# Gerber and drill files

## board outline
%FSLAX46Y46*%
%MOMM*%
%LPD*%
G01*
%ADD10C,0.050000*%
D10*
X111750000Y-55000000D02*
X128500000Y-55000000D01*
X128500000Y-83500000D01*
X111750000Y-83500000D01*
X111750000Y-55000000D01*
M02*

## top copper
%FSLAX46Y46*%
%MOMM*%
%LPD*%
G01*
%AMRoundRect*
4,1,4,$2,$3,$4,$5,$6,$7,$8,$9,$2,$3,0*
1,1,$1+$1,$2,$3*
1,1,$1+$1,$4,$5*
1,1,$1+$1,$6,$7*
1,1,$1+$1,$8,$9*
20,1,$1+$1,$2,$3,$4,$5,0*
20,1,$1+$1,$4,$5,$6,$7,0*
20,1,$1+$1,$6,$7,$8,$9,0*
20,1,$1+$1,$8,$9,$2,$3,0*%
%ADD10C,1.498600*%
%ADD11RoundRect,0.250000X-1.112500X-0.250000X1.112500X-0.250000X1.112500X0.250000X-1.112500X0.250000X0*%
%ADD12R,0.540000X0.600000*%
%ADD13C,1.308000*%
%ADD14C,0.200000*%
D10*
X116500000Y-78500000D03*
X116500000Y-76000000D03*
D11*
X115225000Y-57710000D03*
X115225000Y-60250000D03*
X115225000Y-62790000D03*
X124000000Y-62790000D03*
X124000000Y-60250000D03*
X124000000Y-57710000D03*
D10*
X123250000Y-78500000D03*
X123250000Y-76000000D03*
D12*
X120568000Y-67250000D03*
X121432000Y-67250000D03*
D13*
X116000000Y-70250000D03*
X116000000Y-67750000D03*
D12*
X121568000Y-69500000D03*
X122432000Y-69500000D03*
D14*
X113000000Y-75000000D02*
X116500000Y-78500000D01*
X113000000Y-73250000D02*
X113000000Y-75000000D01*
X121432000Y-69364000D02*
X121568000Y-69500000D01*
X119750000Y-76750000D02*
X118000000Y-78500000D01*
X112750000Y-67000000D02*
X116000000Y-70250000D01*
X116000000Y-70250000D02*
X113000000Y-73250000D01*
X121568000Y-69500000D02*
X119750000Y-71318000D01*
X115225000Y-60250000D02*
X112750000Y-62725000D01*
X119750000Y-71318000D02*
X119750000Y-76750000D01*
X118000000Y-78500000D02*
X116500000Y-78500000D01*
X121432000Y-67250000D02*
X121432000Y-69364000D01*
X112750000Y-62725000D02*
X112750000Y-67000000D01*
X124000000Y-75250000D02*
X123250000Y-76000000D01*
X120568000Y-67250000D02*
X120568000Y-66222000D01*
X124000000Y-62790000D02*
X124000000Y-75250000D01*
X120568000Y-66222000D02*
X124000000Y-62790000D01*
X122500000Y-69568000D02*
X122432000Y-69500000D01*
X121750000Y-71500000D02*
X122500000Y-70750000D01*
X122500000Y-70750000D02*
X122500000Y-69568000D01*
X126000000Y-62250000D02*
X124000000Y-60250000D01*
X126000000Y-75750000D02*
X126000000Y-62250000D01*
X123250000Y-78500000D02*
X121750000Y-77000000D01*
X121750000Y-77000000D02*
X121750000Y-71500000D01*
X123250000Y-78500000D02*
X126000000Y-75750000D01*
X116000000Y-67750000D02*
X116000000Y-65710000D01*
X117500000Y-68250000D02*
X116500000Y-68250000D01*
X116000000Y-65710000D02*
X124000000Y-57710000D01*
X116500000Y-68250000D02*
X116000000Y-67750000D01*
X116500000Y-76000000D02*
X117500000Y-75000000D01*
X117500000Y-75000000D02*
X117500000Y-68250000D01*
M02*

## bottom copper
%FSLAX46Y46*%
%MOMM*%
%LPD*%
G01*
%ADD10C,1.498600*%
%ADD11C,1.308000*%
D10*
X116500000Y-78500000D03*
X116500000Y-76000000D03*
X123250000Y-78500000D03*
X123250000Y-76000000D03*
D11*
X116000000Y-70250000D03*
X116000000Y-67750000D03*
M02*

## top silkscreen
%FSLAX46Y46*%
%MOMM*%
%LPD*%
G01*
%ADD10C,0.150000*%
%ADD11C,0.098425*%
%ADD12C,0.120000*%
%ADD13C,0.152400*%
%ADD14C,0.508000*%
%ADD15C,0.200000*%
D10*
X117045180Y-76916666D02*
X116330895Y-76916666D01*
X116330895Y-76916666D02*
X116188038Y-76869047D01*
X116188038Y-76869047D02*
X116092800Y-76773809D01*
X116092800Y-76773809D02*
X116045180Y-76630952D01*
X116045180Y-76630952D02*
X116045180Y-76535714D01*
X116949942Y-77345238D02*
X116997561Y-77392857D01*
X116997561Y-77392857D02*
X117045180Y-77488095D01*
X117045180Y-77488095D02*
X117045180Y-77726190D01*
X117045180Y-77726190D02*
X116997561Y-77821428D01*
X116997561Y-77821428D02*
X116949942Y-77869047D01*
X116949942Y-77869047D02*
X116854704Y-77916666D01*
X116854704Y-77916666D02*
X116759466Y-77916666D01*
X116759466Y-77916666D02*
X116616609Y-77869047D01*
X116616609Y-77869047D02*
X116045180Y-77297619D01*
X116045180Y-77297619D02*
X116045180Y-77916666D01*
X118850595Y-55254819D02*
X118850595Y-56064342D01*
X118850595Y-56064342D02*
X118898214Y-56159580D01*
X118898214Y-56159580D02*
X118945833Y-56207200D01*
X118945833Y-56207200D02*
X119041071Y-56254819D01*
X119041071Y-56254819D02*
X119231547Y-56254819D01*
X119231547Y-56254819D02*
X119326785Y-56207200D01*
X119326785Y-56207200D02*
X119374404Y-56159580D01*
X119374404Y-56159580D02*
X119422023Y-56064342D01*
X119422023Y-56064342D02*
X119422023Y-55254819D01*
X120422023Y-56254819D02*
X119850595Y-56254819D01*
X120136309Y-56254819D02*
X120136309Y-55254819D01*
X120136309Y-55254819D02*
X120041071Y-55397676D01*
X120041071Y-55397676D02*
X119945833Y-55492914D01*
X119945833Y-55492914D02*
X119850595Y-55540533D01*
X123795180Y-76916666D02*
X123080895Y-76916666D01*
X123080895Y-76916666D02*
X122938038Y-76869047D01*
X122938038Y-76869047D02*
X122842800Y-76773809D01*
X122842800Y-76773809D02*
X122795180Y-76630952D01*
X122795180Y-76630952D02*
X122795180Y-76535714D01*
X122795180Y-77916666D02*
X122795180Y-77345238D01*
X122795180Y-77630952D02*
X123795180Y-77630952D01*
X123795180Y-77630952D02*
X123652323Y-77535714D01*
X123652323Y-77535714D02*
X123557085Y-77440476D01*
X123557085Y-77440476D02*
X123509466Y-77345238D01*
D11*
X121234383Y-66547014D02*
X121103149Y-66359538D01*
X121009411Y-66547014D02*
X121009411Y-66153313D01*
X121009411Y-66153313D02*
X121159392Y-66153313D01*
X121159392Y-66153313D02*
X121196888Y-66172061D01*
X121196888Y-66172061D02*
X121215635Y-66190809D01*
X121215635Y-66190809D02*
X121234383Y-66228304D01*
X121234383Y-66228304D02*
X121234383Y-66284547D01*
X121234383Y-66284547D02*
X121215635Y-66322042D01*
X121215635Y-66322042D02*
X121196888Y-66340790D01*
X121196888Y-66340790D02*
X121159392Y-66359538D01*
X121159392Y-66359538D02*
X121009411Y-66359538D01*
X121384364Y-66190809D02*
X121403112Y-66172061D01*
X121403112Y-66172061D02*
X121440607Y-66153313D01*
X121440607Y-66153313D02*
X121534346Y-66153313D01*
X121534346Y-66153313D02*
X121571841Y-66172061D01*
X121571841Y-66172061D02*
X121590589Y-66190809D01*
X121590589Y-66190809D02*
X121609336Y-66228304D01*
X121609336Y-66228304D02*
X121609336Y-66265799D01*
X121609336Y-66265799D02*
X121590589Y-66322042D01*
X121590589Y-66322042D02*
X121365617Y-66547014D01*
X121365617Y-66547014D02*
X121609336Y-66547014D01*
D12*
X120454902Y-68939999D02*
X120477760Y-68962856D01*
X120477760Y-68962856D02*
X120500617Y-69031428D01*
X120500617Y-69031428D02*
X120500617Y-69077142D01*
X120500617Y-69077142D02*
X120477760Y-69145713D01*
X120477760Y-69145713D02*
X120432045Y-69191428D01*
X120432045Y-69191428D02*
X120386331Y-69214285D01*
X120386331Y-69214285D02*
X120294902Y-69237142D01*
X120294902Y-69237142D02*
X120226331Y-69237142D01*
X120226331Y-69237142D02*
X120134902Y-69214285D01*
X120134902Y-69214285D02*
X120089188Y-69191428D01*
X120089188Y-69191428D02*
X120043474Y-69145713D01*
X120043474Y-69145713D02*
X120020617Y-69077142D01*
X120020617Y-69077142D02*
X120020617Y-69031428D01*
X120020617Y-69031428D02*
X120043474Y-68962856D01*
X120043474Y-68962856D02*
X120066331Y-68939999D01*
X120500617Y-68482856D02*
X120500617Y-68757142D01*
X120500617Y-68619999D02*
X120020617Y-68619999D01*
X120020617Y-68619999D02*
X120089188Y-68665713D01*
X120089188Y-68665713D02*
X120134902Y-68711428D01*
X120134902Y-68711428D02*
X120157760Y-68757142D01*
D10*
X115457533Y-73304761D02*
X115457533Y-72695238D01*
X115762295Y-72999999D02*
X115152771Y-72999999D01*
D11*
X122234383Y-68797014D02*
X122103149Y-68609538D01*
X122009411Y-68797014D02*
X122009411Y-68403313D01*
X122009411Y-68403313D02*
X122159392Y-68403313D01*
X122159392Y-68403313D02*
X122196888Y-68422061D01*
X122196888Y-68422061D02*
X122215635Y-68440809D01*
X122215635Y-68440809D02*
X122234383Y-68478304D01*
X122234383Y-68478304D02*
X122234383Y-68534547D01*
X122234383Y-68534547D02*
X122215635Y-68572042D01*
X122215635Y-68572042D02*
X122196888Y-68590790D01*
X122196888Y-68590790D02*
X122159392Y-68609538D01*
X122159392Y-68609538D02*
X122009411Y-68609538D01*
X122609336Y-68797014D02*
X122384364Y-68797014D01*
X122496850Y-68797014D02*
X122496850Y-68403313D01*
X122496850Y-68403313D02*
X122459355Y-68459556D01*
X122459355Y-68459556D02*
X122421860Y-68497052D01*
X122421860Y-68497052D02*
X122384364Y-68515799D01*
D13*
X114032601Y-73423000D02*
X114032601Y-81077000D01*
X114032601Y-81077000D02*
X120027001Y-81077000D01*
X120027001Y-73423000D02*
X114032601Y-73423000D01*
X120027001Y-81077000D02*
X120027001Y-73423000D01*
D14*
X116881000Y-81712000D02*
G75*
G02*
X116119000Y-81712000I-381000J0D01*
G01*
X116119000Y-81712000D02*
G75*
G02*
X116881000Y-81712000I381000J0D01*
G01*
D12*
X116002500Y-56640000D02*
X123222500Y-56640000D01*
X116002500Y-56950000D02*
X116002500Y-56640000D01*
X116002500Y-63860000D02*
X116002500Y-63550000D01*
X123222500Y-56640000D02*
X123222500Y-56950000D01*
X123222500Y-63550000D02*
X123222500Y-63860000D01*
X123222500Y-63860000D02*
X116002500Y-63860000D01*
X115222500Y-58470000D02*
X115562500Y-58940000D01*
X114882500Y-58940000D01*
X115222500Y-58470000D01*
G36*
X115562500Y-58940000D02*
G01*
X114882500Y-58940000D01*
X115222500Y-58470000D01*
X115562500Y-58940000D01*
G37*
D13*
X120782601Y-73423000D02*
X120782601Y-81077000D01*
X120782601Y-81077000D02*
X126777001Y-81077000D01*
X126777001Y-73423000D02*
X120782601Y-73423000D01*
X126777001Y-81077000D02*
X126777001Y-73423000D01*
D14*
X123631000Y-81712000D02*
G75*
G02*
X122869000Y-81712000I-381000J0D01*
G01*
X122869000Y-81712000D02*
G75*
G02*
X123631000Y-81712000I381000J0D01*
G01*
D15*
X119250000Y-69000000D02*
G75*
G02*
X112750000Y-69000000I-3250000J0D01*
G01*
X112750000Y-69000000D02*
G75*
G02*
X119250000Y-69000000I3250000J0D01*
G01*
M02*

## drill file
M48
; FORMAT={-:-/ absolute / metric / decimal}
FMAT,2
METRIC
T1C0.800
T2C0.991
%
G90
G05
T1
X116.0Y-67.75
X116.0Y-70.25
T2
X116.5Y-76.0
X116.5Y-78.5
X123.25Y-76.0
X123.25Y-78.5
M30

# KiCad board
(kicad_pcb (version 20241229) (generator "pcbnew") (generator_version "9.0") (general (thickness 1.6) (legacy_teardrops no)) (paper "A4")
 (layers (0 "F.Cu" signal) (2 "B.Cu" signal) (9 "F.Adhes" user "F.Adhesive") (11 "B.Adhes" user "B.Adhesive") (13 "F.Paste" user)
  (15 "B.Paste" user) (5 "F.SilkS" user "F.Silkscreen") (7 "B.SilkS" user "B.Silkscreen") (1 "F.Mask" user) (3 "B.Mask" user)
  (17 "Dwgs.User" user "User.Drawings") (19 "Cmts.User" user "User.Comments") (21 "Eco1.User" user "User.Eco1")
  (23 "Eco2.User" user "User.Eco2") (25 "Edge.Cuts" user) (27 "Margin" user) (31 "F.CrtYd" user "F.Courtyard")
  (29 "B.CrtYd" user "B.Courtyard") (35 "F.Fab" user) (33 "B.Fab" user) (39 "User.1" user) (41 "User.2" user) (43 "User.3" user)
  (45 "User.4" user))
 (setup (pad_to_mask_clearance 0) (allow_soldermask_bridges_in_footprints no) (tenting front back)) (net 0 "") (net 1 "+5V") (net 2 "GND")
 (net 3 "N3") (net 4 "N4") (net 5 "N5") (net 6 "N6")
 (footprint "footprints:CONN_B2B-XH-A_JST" (layer "F.Cu") (at 116.5 78.5 -90)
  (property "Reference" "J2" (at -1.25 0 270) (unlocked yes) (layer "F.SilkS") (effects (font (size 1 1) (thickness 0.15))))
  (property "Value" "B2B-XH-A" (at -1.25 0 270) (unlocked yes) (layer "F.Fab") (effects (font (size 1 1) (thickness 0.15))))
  (fp_line (start -5.077 2.467399) (end 2.577 2.467399) (stroke (width 0.1524) (type solid)) (layer "F.SilkS"))
  (fp_line (start 2.577 2.467399) (end 2.577 -3.527001) (stroke (width 0.1524) (type solid)) (layer "F.SilkS"))
  (fp_line (start -5.077 -3.527001) (end -5.077 2.467399) (stroke (width 0.1524) (type solid)) (layer "F.SilkS"))
  (fp_line (start 2.577 -3.527001) (end -5.077 -3.527001) (stroke (width 0.1524) (type solid)) (layer "F.SilkS"))
  (fp_circle (center 3.212 0) (end 3.593 0) (stroke (width 0.508) (type solid)) (fill no) (layer "F.SilkS"))
  (pad "1" thru_hole circle (at 0 0 270) (size 1.4986 1.4986) (drill 0.9906) (layers "*.Cu" "*.Mask") (remove_unused_layers no)
   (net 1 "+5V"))
  (pad "2" thru_hole circle (at -2.5 0 270) (size 1.4986 1.4986) (drill 0.9906) (layers "*.Cu" "*.Mask") (remove_unused_layers no)
   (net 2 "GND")))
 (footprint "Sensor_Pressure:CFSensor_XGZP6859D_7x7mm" (layer "F.Cu") (at 119.6125 60.25)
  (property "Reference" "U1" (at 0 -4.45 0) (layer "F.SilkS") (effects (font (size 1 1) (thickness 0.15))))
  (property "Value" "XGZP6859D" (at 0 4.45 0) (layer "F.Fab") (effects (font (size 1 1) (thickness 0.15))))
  (fp_line (start -3.61 -3.61) (end 3.61 -3.61) (stroke (width 0.12) (type solid)) (layer "F.SilkS"))
  (fp_line (start -3.61 -3.3) (end -3.61 -3.61) (stroke (width 0.12) (type solid)) (layer "F.SilkS"))
  (fp_line (start -3.61 3.61) (end -3.61 3.3) (stroke (width 0.12) (type solid)) (layer "F.SilkS"))
  (fp_line (start 3.61 -3.61) (end 3.61 -3.3) (stroke (width 0.12) (type solid)) (layer "F.SilkS"))
  (fp_line (start 3.61 3.3) (end 3.61 3.61) (stroke (width 0.12) (type solid)) (layer "F.SilkS"))
  (fp_line (start 3.61 3.61) (end -3.61 3.61) (stroke (width 0.12) (type solid)) (layer "F.SilkS"))
  (fp_poly (pts (xy -4.39 -1.78) (xy -4.05 -1.31) (xy -4.73 -1.31)) (stroke (width 0.12) (type solid)) (fill yes) (layer "F.SilkS"))
  (pad "1" smd roundrect (at -4.3875 -2.54) (size 2.725 1) (layers "F.Cu" "F.Mask" "F.Paste") (roundrect_rratio 0.25) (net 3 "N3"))
  (pad "2" smd roundrect (at -4.3875 0) (size 2.725 1) (layers "F.Cu" "F.Mask" "F.Paste") (roundrect_rratio 0.25) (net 1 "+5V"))
  (pad "3" smd roundrect (at -4.3875 2.54) (size 2.725 1) (layers "F.Cu" "F.Mask" "F.Paste") (roundrect_rratio 0.25) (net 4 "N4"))
  (pad "4" smd roundrect (at 4.3875 2.54) (size 2.725 1) (layers "F.Cu" "F.Mask" "F.Paste") (roundrect_rratio 0.25) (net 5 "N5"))
  (pad "5" smd roundrect (at 4.3875 0) (size 2.725 1) (layers "F.Cu" "F.Mask" "F.Paste") (roundrect_rratio 0.25) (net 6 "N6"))
  (pad "6" smd roundrect (at 4.3875 -2.54) (size 2.725 1) (layers "F.Cu" "F.Mask" "F.Paste") (roundrect_rratio 0.25) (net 2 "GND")))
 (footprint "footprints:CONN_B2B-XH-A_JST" (layer "F.Cu") (at 123.25 78.5 -90)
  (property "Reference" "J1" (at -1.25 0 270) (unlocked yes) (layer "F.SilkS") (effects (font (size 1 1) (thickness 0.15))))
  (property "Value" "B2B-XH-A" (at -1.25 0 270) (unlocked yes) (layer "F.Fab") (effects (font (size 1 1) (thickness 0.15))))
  (fp_line (start -5.077 2.467399) (end 2.577 2.467399) (stroke (width 0.1524) (type solid)) (layer "F.SilkS"))
  (fp_line (start 2.577 2.467399) (end 2.577 -3.527001) (stroke (width 0.1524) (type solid)) (layer "F.SilkS"))
  (fp_line (start -5.077 -3.527001) (end -5.077 2.467399) (stroke (width 0.1524) (type solid)) (layer "F.SilkS"))
  (fp_line (start 2.577 -3.527001) (end -5.077 -3.527001) (stroke (width 0.1524) (type solid)) (layer "F.SilkS"))
  (fp_circle (center 3.212 0) (end 3.593 0) (stroke (width 0.508) (type solid)) (fill no) (layer "F.SilkS"))
  (pad "1" thru_hole circle (at 0 0 270) (size 1.4986 1.4986) (drill 0.9906) (layers "*.Cu" "*.Mask") (remove_unused_layers no) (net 6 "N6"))
  (pad "2" thru_hole circle (at -2.5 0 270) (size 1.4986 1.4986) (drill 0.9906) (layers "*.Cu" "*.Mask") (remove_unused_layers no)
   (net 5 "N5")))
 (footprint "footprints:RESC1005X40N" (layer "F.Cu") (at 121 67.25)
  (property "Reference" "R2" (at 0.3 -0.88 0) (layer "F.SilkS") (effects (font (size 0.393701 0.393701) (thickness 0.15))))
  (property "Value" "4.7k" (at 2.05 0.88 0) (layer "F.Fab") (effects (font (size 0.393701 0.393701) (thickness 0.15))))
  (pad "1" smd rect (at -0.432 0) (size 0.54 0.6) (layers "F.Cu" "F.Mask" "F.Paste") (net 5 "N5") (solder_mask_margin 0.102))
  (pad "2" smd rect (at 0.432 0) (size 0.54 0.6) (layers "F.Cu" "F.Mask" "F.Paste") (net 1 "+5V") (solder_mask_margin 0.102)))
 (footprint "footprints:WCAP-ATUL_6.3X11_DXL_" (layer "F.Cu") (at 116 69 -90)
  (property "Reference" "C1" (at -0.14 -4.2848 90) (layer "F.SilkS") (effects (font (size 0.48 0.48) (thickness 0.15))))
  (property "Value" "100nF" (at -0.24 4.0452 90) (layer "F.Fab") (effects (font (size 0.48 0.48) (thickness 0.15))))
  (fp_circle (center 0 0) (end 3.25 0) (stroke (width 0.2) (type solid)) (fill no) (layer "F.SilkS"))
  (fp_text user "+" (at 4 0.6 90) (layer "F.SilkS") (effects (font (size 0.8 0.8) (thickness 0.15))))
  (pad "1" thru_hole circle (at 1.25 0 270) (size 1.308 1.308) (drill 0.8) (layers "*.Cu" "*.Mask") (remove_unused_layers no) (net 1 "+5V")
   (solder_mask_margin 0.102))
  (pad "2" thru_hole circle (at -1.25 0 270) (size 1.308 1.308) (drill 0.8) (layers "*.Cu" "*.Mask") (remove_unused_layers no) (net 2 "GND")
   (solder_mask_margin 0.102)))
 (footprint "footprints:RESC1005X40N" (layer "F.Cu") (at 122 69.5)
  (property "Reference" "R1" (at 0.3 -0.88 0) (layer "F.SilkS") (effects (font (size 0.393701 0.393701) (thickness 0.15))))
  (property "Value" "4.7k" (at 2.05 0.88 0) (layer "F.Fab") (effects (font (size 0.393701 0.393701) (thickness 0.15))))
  (pad "1" smd rect (at -0.432 0) (size 0.54 0.6) (layers "F.Cu" "F.Mask" "F.Paste") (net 1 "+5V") (solder_mask_margin 0.102))
  (pad "2" smd rect (at 0.432 0) (size 0.54 0.6) (layers "F.Cu" "F.Mask" "F.Paste") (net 6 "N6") (solder_mask_margin 0.102)))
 (gr_rect (start 111.75 55) (end 128.5 83.5) (stroke (width 0.05) (type default)) (fill no) (layer "Edge.Cuts"))
 (segment (start 113 75) (end 116.5 78.5) (width 0.2) (layer "F.Cu") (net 1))
 (segment (start 113 73.25) (end 113 75) (width 0.2) (layer "F.Cu") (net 1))
 (segment (start 121.432 69.364) (end 121.568 69.5) (width 0.2) (layer "F.Cu") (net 1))
 (segment (start 119.75 76.75) (end 118 78.5) (width 0.2) (layer "F.Cu") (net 1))
 (segment (start 112.75 67) (end 116 70.25) (width 0.2) (layer "F.Cu") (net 1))
 (segment (start 116 70.25) (end 113 73.25) (width 0.2) (layer "F.Cu") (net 1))
 (segment (start 121.568 69.5) (end 119.75 71.318) (width 0.2) (layer "F.Cu") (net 1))
 (segment (start 115.225 60.25) (end 112.75 62.725) (width 0.2) (layer "F.Cu") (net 1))
 (segment (start 119.75 71.318) (end 119.75 76.75) (width 0.2) (layer "F.Cu") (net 1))
 (segment (start 118 78.5) (end 116.5 78.5) (width 0.2) (layer "F.Cu") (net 1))
 (segment (start 121.432 67.25) (end 121.432 69.364) (width 0.2) (layer "F.Cu") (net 1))
 (segment (start 112.75 62.725) (end 112.75 67) (width 0.2) (layer "F.Cu") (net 1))
 (segment (start 124 75.25) (end 123.25 76) (width 0.2) (layer "F.Cu") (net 5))
 (segment (start 120.568 67.25) (end 120.568 66.222) (width 0.2) (layer "F.Cu") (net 5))
 (segment (start 124 62.79) (end 124 75.25) (width 0.2) (layer "F.Cu") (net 5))
 (segment (start 120.568 66.222) (end 124 62.79) (width 0.2) (layer "F.Cu") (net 5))
 (segment (start 122.5 69.568) (end 122.432 69.5) (width 0.2) (layer "F.Cu") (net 6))
 (segment (start 121.75 71.5) (end 122.5 70.75) (width 0.2) (layer "F.Cu") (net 6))
 (segment (start 122.5 70.75) (end 122.5 69.568) (width 0.2) (layer "F.Cu") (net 6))
 (segment (start 126 62.25) (end 124 60.25) (width 0.2) (layer "F.Cu") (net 6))
 (segment (start 126 75.75) (end 126 62.25) (width 0.2) (layer "F.Cu") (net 6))
 (segment (start 123.25 78.5) (end 121.75 77) (width 0.2) (layer "F.Cu") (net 6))
 (segment (start 121.75 77) (end 121.75 71.5) (width 0.2) (layer "F.Cu") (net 6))
 (segment (start 123.25 78.5) (end 126 75.75) (width 0.2) (layer "F.Cu") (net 6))
 (segment (start 116 67.75) (end 116 65.71) (width 0.2) (layer "F.Cu") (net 2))
 (segment (start 117.5 68.25) (end 116.5 68.25) (width 0.2) (layer "F.Cu") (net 2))
 (segment (start 116 65.71) (end 124 57.71) (width 0.2) (layer "F.Cu") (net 2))
 (segment (start 116.5 68.25) (end 116 67.75) (width 0.2) (layer "F.Cu") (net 2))
 (segment (start 116.5 76) (end 117.5 75) (width 0.2) (layer "F.Cu") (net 2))
 (segment (start 117.5 75) (end 117.5 68.25) (width 0.2) (layer "F.Cu") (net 2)))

